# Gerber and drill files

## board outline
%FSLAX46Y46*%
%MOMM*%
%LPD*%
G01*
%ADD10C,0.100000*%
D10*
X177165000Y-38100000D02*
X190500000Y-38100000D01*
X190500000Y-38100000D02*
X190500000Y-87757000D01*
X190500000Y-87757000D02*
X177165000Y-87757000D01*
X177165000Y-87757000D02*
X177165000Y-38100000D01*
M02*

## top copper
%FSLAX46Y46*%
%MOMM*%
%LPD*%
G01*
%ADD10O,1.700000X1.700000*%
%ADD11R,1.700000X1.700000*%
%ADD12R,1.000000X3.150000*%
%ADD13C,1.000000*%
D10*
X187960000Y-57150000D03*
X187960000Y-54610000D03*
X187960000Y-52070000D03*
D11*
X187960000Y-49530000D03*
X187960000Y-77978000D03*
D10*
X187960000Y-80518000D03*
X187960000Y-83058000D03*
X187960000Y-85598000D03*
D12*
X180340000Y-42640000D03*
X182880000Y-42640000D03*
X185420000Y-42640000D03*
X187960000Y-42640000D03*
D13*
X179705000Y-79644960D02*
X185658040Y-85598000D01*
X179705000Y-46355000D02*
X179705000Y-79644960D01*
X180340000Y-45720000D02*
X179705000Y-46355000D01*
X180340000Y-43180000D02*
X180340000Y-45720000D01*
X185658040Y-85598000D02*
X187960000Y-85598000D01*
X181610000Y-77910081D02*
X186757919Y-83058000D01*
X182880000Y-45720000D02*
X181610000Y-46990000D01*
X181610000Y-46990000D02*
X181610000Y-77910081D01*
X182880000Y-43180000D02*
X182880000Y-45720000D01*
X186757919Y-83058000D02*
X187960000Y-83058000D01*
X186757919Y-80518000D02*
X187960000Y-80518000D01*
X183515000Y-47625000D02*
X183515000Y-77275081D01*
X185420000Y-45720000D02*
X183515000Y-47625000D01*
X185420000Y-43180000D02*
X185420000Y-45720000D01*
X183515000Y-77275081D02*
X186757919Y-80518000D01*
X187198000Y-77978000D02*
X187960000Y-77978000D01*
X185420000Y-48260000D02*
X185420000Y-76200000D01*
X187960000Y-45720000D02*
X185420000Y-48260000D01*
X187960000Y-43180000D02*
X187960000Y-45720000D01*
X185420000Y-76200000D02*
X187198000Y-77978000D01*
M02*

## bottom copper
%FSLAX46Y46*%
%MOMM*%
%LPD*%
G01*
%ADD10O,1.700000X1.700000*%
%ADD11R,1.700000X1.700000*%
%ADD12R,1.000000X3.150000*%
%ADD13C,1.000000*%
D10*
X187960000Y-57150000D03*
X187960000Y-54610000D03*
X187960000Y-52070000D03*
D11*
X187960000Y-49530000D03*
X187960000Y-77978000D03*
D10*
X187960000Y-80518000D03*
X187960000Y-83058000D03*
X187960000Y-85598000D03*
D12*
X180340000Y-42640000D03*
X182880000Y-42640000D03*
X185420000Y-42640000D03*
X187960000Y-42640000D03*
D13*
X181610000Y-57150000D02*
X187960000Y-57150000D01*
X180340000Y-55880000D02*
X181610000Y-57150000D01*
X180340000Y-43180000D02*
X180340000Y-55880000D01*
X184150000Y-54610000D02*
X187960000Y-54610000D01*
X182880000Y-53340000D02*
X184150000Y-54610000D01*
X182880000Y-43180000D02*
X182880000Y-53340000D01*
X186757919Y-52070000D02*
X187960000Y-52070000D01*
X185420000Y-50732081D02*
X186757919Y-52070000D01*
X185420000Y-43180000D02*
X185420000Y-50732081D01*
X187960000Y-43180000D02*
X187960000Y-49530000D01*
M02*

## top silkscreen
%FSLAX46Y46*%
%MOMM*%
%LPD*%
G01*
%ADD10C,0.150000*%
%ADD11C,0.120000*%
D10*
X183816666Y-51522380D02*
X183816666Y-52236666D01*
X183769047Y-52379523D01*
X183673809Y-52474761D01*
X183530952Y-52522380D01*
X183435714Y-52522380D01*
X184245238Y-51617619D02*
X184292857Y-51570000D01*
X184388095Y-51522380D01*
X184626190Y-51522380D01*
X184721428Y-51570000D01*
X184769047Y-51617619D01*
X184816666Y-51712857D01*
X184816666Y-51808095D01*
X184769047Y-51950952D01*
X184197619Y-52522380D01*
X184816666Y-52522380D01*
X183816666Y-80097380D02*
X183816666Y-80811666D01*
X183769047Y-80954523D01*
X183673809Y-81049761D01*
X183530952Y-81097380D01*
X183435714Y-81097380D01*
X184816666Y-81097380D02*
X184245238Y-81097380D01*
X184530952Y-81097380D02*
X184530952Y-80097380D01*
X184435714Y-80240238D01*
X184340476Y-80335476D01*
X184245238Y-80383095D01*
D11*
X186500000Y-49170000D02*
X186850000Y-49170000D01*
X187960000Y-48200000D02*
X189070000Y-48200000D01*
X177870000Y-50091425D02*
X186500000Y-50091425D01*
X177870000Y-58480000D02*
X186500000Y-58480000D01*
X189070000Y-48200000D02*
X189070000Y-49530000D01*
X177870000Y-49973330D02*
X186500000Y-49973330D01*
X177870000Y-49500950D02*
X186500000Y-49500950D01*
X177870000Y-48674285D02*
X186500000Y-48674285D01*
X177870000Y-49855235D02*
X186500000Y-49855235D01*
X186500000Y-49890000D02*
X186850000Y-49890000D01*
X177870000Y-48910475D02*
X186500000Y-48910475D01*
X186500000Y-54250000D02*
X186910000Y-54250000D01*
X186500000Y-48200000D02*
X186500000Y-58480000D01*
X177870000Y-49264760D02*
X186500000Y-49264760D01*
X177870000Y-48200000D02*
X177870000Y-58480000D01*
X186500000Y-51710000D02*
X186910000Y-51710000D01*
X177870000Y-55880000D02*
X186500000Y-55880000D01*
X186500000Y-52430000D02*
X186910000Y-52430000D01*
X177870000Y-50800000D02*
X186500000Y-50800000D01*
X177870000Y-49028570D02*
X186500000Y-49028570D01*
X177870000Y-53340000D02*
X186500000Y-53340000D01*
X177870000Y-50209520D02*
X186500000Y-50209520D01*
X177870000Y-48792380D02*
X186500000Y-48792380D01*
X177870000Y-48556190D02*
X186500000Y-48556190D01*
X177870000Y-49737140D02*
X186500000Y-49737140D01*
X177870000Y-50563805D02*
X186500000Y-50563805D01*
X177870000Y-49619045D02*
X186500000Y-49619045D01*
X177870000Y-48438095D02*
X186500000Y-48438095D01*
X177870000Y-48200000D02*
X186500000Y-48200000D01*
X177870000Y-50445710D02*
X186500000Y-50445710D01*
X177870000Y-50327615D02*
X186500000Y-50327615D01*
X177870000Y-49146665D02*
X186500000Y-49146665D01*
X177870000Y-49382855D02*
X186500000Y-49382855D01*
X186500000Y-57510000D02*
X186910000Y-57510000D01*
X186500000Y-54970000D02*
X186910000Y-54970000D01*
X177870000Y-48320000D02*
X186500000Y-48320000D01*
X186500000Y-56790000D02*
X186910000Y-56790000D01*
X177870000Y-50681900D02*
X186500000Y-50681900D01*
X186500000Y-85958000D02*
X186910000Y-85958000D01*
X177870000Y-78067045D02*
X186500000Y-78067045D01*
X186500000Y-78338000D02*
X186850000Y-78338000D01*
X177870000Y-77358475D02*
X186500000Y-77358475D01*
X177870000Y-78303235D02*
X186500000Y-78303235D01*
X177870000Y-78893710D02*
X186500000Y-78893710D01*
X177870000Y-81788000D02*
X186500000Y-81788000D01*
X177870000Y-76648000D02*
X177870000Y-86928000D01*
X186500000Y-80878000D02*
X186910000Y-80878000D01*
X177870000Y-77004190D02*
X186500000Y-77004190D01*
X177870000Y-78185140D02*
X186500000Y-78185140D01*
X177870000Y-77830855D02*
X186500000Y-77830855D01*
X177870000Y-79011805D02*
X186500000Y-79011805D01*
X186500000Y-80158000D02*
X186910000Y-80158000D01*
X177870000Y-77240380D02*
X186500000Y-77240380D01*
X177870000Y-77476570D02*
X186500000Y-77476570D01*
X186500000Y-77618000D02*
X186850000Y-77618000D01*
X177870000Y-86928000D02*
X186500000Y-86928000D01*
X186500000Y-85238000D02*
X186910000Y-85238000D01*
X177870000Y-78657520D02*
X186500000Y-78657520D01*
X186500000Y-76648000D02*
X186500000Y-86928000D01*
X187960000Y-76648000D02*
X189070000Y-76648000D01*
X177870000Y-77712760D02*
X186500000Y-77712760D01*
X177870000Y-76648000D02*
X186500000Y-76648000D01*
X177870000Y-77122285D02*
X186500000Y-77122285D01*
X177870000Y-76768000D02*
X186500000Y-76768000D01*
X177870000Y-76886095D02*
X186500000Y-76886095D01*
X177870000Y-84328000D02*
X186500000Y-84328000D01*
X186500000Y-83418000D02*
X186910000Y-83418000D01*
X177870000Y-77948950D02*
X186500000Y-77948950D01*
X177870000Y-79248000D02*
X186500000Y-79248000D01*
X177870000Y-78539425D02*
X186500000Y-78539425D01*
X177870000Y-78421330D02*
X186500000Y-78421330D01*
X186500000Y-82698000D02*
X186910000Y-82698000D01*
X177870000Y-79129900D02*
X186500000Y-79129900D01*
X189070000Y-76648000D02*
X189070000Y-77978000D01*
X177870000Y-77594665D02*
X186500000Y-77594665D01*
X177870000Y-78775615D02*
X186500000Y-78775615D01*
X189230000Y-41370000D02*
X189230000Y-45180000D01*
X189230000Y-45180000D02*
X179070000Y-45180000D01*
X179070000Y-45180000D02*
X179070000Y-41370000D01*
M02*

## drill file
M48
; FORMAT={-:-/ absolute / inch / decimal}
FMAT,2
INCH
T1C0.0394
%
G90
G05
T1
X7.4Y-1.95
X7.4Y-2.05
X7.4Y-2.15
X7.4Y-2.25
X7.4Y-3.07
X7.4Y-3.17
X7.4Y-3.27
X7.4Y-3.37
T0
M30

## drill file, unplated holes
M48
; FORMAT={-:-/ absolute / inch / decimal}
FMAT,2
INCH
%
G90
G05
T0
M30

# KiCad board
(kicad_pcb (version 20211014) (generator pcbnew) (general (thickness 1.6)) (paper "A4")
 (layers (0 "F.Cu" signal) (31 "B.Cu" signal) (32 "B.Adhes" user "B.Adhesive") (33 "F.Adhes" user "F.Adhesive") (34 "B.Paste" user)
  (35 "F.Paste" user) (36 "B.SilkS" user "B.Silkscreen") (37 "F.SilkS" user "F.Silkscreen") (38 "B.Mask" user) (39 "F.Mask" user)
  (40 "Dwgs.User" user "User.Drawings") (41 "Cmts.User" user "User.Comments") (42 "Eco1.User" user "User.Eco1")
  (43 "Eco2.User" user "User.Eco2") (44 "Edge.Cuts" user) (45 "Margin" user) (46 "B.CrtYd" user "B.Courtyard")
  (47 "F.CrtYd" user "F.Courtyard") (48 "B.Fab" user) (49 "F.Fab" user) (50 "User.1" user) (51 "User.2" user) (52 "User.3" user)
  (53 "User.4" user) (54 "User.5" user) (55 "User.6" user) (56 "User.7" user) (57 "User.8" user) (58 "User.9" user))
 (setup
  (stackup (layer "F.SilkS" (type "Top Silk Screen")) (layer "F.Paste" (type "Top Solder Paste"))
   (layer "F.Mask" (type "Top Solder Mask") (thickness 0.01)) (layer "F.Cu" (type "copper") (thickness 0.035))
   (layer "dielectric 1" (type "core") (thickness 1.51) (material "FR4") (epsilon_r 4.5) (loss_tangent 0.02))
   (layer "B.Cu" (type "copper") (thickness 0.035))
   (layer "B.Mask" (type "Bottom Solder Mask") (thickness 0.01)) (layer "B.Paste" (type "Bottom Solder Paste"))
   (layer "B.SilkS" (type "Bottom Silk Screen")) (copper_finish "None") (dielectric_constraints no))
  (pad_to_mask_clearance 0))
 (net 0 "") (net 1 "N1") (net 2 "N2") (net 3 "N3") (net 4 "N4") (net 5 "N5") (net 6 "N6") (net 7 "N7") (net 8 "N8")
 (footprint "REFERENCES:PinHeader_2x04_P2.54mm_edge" (layer "F.Cu") (at 184.15 40.1 -90)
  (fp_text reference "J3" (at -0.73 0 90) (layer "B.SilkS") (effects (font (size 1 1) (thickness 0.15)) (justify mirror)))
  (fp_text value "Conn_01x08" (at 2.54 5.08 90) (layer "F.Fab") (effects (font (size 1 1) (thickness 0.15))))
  (fp_line (start 5.08 5.08) (end 1.27 5.08) (layer "F.SilkS") (width 0.12))
  (fp_line (start 5.08 -5.08) (end 5.08 5.08) (layer "F.SilkS") (width 0.12))
  (fp_line (start 1.27 -5.08) (end 5.08 -5.08) (layer "F.SilkS") (width 0.12))
  (pad "1" smd rect (at 2.54 -3.81 270) (size 3.15 1) (layers "F.Cu" "F.Paste" "F.Mask") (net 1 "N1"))
  (pad "2" smd rect (at 2.54 -1.27 270) (size 3.15 1) (layers "F.Cu" "F.Paste" "F.Mask") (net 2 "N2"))
  (pad "3" smd rect (at 2.54 1.27 270) (size 3.15 1) (layers "F.Cu" "F.Paste" "F.Mask") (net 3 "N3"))
  (pad "4" smd rect (at 2.54 3.81 270) (size 3.15 1) (layers "F.Cu" "F.Paste" "F.Mask") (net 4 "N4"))
  (pad "5" smd rect (at 2.54 -3.81 270) (size 3.15 1) (layers "B.Cu" "B.Paste" "B.Mask") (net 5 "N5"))
  (pad "6" smd rect (at 2.54 -1.27 270) (size 3.15 1) (layers "B.Cu" "B.Paste" "B.Mask") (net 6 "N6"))
  (pad "7" smd rect (at 2.54 1.27 270) (size 3.15 1) (layers "B.Cu" "B.Paste" "B.Mask") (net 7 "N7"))
  (pad "8" smd rect (at 2.54 3.81 270) (size 3.15 1) (layers "B.Cu" "B.Paste" "B.Mask") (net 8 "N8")))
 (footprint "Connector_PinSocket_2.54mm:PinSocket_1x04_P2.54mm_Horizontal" (layer "F.Cu") (at 187.96 49.53)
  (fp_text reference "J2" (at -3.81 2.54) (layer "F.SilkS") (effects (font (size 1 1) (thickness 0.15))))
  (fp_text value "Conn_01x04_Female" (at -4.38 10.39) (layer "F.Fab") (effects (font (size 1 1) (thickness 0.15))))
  (fp_line (start -10.09 1.1519) (end -1.46 1.1519) (layer "F.SilkS") (width 0.12))
  (fp_line (start -1.46 7.26) (end -1.05 7.26) (layer "F.SilkS") (width 0.12))
  (fp_line (start -10.09 -1.21) (end -1.46 -1.21) (layer "F.SilkS") (width 0.12))
  (fp_line (start -1.46 5.44) (end -1.05 5.44) (layer "F.SilkS") (width 0.12))
  (fp_line (start -1.46 7.98) (end -1.05 7.98) (layer "F.SilkS") (width 0.12))
  (fp_line (start -10.09 -0.147145) (end -1.46 -0.147145) (layer "F.SilkS") (width 0.12))
  (fp_line (start -10.09 -0.383335) (end -1.46 -0.383335) (layer "F.SilkS") (width 0.12))
  (fp_line (start -10.09 0.797615) (end -1.46 0.797615) (layer "F.SilkS") (width 0.12))
  (fp_line (start -10.09 0.91571) (end -1.46 0.91571) (layer "F.SilkS") (width 0.12))
  (fp_line (start -10.09 -1.33) (end -1.46 -1.33) (layer "F.SilkS") (width 0.12))
  (fp_line (start -10.09 -1.091905) (end -1.46 -1.091905) (layer "F.SilkS") (width 0.12))
  (fp_line (start -10.09 0.089045) (end -1.46 0.089045) (layer "F.SilkS") (width 0.12))
  (fp_line (start -10.09 1.033805) (end -1.46 1.033805) (layer "F.SilkS") (width 0.12))
  (fp_line (start -10.09 0.20714) (end -1.46 0.20714) (layer "F.SilkS") (width 0.12))
  (fp_line (start -10.09 -0.97381) (end -1.46 -0.97381) (layer "F.SilkS") (width 0.12))
  (fp_line (start -10.09 -0.73762) (end -1.46 -0.73762) (layer "F.SilkS") (width 0.12))
  (fp_line (start -10.09 0.67952) (end -1.46 0.67952) (layer "F.SilkS") (width 0.12))
  (fp_line (start -10.09 3.81) (end -1.46 3.81) (layer "F.SilkS") (width 0.12))
  (fp_line (start -10.09 -0.50143) (end -1.46 -0.50143) (layer "F.SilkS") (width 0.12))
  (fp_line (start -10.09 1.27) (end -1.46 1.27) (layer "F.SilkS") (width 0.12))
  (fp_line (start -1.46 2.9) (end -1.05 2.9) (layer "F.SilkS") (width 0.12))
  (fp_line (start -10.09 6.35) (end -1.46 6.35) (layer "F.SilkS") (width 0.12))
  (fp_line (start -1.46 2.18) (end -1.05 2.18) (layer "F.SilkS") (width 0.12))
  (fp_line (start -10.09 -1.33) (end -10.09 8.95) (layer "F.SilkS") (width 0.12))
  (fp_line (start -10.09 -0.26524) (end -1.46 -0.26524) (layer "F.SilkS") (width 0.12))
  (fp_line (start -1.46 -1.33) (end -1.46 8.95) (layer "F.SilkS") (width 0.12))
  (fp_line (start -1.46 4.72) (end -1.05 4.72) (layer "F.SilkS") (width 0.12))
  (fp_line (start -10.09 -0.619525) (end -1.46 -0.619525) (layer "F.SilkS") (width 0.12))
  (fp_line (start -1.46 0.36) (end -1.11 0.36) (layer "F.SilkS") (width 0.12))
  (fp_line (start -10.09 0.325235) (end -1.46 0.325235) (layer "F.SilkS") (width 0.12))
  (fp_line (start -10.09 -0.855715) (end -1.46 -0.855715) (layer "F.SilkS") (width 0.12))
  (fp_line (start -10.09 -0.02905) (end -1.46 -0.02905) (layer "F.SilkS") (width 0.12))
  (fp_line (start -10.09 0.44333) (end -1.46 0.44333) (layer "F.SilkS") (width 0.12))
  (fp_line (start 1.11 -1.33) (end 1.11 0) (layer "F.SilkS") (width 0.12))
  (fp_line (start -10.09 8.95) (end -1.46 8.95) (layer "F.SilkS") (width 0.12))
  (fp_line (start -10.09 0.561425) (end -1.46 0.561425) (layer "F.SilkS") (width 0.12))
  (fp_line (start 0 -1.33) (end 1.11 -1.33) (layer "F.SilkS") (width 0.12))
  (fp_line (start -1.46 -0.36) (end -1.11 -0.36) (layer "F.SilkS") (width 0.12))
  (pad "1" thru_hole rect (at 0 0) (size 1.7 1.7) (drill 1) (layers *.Cu *.Mask) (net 5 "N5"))
  (pad "2" thru_hole oval (at 0 2.54) (size 1.7 1.7) (drill 1) (layers *.Cu *.Mask) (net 6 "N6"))
  (pad "3" thru_hole oval (at 0 5.08) (size 1.7 1.7) (drill 1) (layers *.Cu *.Mask) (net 7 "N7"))
  (pad "4" thru_hole oval (at 0 7.62) (size 1.7 1.7) (drill 1) (layers *.Cu *.Mask) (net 8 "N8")))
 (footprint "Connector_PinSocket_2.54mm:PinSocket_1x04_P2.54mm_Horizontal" (layer "F.Cu") (at 187.96 77.978)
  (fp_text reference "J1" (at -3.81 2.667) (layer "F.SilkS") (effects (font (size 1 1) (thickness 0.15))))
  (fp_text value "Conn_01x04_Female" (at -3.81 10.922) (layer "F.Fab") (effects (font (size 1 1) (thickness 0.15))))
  (fp_line (start -1.46 7.98) (end -1.05 7.98) (layer "F.SilkS") (width 0.12))
  (fp_line (start -10.09 0.089045) (end -1.46 0.089045) (layer "F.SilkS") (width 0.12))
  (fp_line (start -1.46 0.36) (end -1.11 0.36) (layer "F.SilkS") (width 0.12))
  (fp_line (start -10.09 -0.619525) (end -1.46 -0.619525) (layer "F.SilkS") (width 0.12))
  (fp_line (start -10.09 0.325235) (end -1.46 0.325235) (layer "F.SilkS") (width 0.12))
  (fp_line (start -10.09 0.91571) (end -1.46 0.91571) (layer "F.SilkS") (width 0.12))
  (fp_line (start -10.09 3.81) (end -1.46 3.81) (layer "F.SilkS") (width 0.12))
  (fp_line (start -10.09 -1.33) (end -10.09 8.95) (layer "F.SilkS") (width 0.12))
  (fp_line (start -1.46 2.9) (end -1.05 2.9) (layer "F.SilkS") (width 0.12))
  (fp_line (start -10.09 -0.97381) (end -1.46 -0.97381) (layer "F.SilkS") (width 0.12))
  (fp_line (start -10.09 0.20714) (end -1.46 0.20714) (layer "F.SilkS") (width 0.12))
  (fp_line (start -10.09 -0.147145) (end -1.46 -0.147145) (layer "F.SilkS") (width 0.12))
  (fp_line (start -10.09 1.033805) (end -1.46 1.033805) (layer "F.SilkS") (width 0.12))
  (fp_line (start -1.46 2.18) (end -1.05 2.18) (layer "F.SilkS") (width 0.12))
  (fp_line (start -10.09 -0.73762) (end -1.46 -0.73762) (layer "F.SilkS") (width 0.12))
  (fp_line (start -10.09 -0.50143) (end -1.46 -0.50143) (layer "F.SilkS") (width 0.12))
  (fp_line (start -1.46 -0.36) (end -1.11 -0.36) (layer "F.SilkS") (width 0.12))
  (fp_line (start -10.09 8.95) (end -1.46 8.95) (layer "F.SilkS") (width 0.12))
  (fp_line (start -1.46 7.26) (end -1.05 7.26) (layer "F.SilkS") (width 0.12))
  (fp_line (start -10.09 0.67952) (end -1.46 0.67952) (layer "F.SilkS") (width 0.12))
  (fp_line (start -1.46 -1.33) (end -1.46 8.95) (layer "F.SilkS") (width 0.12))
  (fp_line (start 0 -1.33) (end 1.11 -1.33) (layer "F.SilkS") (width 0.12))
  (fp_line (start -10.09 -0.26524) (end -1.46 -0.26524) (layer "F.SilkS") (width 0.12))
  (fp_line (start -10.09 -1.33) (end -1.46 -1.33) (layer "F.SilkS") (width 0.12))
  (fp_line (start -10.09 -0.855715) (end -1.46 -0.855715) (layer "F.SilkS") (width 0.12))
  (fp_line (start -10.09 -1.21) (end -1.46 -1.21) (layer "F.SilkS") (width 0.12))
  (fp_line (start -10.09 -1.091905) (end -1.46 -1.091905) (layer "F.SilkS") (width 0.12))
  (fp_line (start -10.09 6.35) (end -1.46 6.35) (layer "F.SilkS") (width 0.12))
  (fp_line (start -1.46 5.44) (end -1.05 5.44) (layer "F.SilkS") (width 0.12))
  (fp_line (start -10.09 -0.02905) (end -1.46 -0.02905) (layer "F.SilkS") (width 0.12))
  (fp_line (start -10.09 1.27) (end -1.46 1.27) (layer "F.SilkS") (width 0.12))
  (fp_line (start -10.09 0.561425) (end -1.46 0.561425) (layer "F.SilkS") (width 0.12))
  (fp_line (start -10.09 0.44333) (end -1.46 0.44333) (layer "F.SilkS") (width 0.12))
  (fp_line (start -1.46 4.72) (end -1.05 4.72) (layer "F.SilkS") (width 0.12))
  (fp_line (start -10.09 1.1519) (end -1.46 1.1519) (layer "F.SilkS") (width 0.12))
  (fp_line (start 1.11 -1.33) (end 1.11 0) (layer "F.SilkS") (width 0.12))
  (fp_line (start -10.09 -0.383335) (end -1.46 -0.383335) (layer "F.SilkS") (width 0.12))
  (fp_line (start -10.09 0.797615) (end -1.46 0.797615) (layer "F.SilkS") (width 0.12))
  (pad "1" thru_hole rect (at 0 0) (size 1.7 1.7) (drill 1) (layers *.Cu *.Mask) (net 1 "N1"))
  (pad "2" thru_hole oval (at 0 2.54) (size 1.7 1.7) (drill 1) (layers *.Cu *.Mask) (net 2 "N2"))
  (pad "3" thru_hole oval (at 0 5.08) (size 1.7 1.7) (drill 1) (layers *.Cu *.Mask) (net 3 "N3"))
  (pad "4" thru_hole oval (at 0 7.62) (size 1.7 1.7) (drill 1) (layers *.Cu *.Mask) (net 4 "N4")))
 (gr_rect (start 177.165 38.1) (end 190.5 87.757) (layer "Edge.Cuts") (width 0.1) (fill none))
 (segment (start 187.96 43.18) (end 187.96 45.72) (width 1) (layer "F.Cu") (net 1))
 (segment (start 185.42 48.26) (end 185.42 76.2) (width 1) (layer "F.Cu") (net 1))
 (segment (start 185.42 76.2) (end 187.198 77.978) (width 1) (layer "F.Cu") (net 1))
 (segment (start 187.96 45.72) (end 185.42 48.26) (width 1) (layer "F.Cu") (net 1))
 (segment (start 187.198 77.978) (end 187.96 77.978) (width 1) (layer "F.Cu") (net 1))
 (segment (start 183.515 47.625) (end 183.515 77.275081) (width 1) (layer "F.Cu") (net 2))
 (segment (start 186.757919 80.518) (end 187.96 80.518) (width 1) (layer "F.Cu") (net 2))
 (segment (start 183.515 77.275081) (end 186.757919 80.518) (width 1) (layer "F.Cu") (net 2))
 (segment (start 185.42 45.72) (end 183.515 47.625) (width 1) (layer "F.Cu") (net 2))
 (segment (start 185.42 43.18) (end 185.42 45.72) (width 1) (layer "F.Cu") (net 2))
 (segment (start 182.88 43.18) (end 182.88 45.72) (width 1) (layer "F.Cu") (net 3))
 (segment (start 181.61 77.910081) (end 186.757919 83.058) (width 1) (layer "F.Cu") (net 3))
 (segment (start 182.88 45.72) (end 181.61 46.99) (width 1) (layer "F.Cu") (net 3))
 (segment (start 186.757919 83.058) (end 187.96 83.058) (width 1) (layer "F.Cu") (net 3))
 (segment (start 181.61 46.99) (end 181.61 77.910081) (width 1) (layer "F.Cu") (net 3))
 (segment (start 179.705 46.355) (end 179.705 79.64496) (width 1) (layer "F.Cu") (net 4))
 (segment (start 179.705 79.64496) (end 185.65804 85.598) (width 1) (layer "F.Cu") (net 4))
 (segment (start 180.34 43.18) (end 180.34 45.72) (width 1) (layer "F.Cu") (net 4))
 (segment (start 180.34 45.72) (end 179.705 46.355) (width 1) (layer "F.Cu") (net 4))
 (segment (start 185.65804 85.598) (end 187.96 85.598) (width 1) (layer "F.Cu") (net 4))
 (segment (start 187.96 43.18) (end 187.96 49.53) (width 1) (layer "B.Cu") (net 5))
 (segment (start 185.42 43.18) (end 185.42 50.732081) (width 1) (layer "B.Cu") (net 6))
 (segment (start 185.42 50.732081) (end 186.757919 52.07) (width 1) (layer "B.Cu") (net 6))
 (segment (start 186.757919 52.07) (end 187.96 52.07) (width 1) (layer "B.Cu") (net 6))
 (segment (start 182.88 53.34) (end 184.15 54.61) (width 1) (layer "B.Cu") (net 7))
 (segment (start 182.88 43.18) (end 182.88 53.34) (width 1) (layer "B.Cu") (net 7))
 (segment (start 184.15 54.61) (end 187.96 54.61) (width 1) (layer "B.Cu") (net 7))
 (segment (start 180.34 55.88) (end 181.61 57.15) (width 1) (layer "B.Cu") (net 8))
 (segment (start 180.34 43.18) (end 180.34 55.88) (width 1) (layer "B.Cu") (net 8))
 (segment (start 181.61 57.15) (end 187.96 57.15) (width 1) (layer "B.Cu") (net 8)))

